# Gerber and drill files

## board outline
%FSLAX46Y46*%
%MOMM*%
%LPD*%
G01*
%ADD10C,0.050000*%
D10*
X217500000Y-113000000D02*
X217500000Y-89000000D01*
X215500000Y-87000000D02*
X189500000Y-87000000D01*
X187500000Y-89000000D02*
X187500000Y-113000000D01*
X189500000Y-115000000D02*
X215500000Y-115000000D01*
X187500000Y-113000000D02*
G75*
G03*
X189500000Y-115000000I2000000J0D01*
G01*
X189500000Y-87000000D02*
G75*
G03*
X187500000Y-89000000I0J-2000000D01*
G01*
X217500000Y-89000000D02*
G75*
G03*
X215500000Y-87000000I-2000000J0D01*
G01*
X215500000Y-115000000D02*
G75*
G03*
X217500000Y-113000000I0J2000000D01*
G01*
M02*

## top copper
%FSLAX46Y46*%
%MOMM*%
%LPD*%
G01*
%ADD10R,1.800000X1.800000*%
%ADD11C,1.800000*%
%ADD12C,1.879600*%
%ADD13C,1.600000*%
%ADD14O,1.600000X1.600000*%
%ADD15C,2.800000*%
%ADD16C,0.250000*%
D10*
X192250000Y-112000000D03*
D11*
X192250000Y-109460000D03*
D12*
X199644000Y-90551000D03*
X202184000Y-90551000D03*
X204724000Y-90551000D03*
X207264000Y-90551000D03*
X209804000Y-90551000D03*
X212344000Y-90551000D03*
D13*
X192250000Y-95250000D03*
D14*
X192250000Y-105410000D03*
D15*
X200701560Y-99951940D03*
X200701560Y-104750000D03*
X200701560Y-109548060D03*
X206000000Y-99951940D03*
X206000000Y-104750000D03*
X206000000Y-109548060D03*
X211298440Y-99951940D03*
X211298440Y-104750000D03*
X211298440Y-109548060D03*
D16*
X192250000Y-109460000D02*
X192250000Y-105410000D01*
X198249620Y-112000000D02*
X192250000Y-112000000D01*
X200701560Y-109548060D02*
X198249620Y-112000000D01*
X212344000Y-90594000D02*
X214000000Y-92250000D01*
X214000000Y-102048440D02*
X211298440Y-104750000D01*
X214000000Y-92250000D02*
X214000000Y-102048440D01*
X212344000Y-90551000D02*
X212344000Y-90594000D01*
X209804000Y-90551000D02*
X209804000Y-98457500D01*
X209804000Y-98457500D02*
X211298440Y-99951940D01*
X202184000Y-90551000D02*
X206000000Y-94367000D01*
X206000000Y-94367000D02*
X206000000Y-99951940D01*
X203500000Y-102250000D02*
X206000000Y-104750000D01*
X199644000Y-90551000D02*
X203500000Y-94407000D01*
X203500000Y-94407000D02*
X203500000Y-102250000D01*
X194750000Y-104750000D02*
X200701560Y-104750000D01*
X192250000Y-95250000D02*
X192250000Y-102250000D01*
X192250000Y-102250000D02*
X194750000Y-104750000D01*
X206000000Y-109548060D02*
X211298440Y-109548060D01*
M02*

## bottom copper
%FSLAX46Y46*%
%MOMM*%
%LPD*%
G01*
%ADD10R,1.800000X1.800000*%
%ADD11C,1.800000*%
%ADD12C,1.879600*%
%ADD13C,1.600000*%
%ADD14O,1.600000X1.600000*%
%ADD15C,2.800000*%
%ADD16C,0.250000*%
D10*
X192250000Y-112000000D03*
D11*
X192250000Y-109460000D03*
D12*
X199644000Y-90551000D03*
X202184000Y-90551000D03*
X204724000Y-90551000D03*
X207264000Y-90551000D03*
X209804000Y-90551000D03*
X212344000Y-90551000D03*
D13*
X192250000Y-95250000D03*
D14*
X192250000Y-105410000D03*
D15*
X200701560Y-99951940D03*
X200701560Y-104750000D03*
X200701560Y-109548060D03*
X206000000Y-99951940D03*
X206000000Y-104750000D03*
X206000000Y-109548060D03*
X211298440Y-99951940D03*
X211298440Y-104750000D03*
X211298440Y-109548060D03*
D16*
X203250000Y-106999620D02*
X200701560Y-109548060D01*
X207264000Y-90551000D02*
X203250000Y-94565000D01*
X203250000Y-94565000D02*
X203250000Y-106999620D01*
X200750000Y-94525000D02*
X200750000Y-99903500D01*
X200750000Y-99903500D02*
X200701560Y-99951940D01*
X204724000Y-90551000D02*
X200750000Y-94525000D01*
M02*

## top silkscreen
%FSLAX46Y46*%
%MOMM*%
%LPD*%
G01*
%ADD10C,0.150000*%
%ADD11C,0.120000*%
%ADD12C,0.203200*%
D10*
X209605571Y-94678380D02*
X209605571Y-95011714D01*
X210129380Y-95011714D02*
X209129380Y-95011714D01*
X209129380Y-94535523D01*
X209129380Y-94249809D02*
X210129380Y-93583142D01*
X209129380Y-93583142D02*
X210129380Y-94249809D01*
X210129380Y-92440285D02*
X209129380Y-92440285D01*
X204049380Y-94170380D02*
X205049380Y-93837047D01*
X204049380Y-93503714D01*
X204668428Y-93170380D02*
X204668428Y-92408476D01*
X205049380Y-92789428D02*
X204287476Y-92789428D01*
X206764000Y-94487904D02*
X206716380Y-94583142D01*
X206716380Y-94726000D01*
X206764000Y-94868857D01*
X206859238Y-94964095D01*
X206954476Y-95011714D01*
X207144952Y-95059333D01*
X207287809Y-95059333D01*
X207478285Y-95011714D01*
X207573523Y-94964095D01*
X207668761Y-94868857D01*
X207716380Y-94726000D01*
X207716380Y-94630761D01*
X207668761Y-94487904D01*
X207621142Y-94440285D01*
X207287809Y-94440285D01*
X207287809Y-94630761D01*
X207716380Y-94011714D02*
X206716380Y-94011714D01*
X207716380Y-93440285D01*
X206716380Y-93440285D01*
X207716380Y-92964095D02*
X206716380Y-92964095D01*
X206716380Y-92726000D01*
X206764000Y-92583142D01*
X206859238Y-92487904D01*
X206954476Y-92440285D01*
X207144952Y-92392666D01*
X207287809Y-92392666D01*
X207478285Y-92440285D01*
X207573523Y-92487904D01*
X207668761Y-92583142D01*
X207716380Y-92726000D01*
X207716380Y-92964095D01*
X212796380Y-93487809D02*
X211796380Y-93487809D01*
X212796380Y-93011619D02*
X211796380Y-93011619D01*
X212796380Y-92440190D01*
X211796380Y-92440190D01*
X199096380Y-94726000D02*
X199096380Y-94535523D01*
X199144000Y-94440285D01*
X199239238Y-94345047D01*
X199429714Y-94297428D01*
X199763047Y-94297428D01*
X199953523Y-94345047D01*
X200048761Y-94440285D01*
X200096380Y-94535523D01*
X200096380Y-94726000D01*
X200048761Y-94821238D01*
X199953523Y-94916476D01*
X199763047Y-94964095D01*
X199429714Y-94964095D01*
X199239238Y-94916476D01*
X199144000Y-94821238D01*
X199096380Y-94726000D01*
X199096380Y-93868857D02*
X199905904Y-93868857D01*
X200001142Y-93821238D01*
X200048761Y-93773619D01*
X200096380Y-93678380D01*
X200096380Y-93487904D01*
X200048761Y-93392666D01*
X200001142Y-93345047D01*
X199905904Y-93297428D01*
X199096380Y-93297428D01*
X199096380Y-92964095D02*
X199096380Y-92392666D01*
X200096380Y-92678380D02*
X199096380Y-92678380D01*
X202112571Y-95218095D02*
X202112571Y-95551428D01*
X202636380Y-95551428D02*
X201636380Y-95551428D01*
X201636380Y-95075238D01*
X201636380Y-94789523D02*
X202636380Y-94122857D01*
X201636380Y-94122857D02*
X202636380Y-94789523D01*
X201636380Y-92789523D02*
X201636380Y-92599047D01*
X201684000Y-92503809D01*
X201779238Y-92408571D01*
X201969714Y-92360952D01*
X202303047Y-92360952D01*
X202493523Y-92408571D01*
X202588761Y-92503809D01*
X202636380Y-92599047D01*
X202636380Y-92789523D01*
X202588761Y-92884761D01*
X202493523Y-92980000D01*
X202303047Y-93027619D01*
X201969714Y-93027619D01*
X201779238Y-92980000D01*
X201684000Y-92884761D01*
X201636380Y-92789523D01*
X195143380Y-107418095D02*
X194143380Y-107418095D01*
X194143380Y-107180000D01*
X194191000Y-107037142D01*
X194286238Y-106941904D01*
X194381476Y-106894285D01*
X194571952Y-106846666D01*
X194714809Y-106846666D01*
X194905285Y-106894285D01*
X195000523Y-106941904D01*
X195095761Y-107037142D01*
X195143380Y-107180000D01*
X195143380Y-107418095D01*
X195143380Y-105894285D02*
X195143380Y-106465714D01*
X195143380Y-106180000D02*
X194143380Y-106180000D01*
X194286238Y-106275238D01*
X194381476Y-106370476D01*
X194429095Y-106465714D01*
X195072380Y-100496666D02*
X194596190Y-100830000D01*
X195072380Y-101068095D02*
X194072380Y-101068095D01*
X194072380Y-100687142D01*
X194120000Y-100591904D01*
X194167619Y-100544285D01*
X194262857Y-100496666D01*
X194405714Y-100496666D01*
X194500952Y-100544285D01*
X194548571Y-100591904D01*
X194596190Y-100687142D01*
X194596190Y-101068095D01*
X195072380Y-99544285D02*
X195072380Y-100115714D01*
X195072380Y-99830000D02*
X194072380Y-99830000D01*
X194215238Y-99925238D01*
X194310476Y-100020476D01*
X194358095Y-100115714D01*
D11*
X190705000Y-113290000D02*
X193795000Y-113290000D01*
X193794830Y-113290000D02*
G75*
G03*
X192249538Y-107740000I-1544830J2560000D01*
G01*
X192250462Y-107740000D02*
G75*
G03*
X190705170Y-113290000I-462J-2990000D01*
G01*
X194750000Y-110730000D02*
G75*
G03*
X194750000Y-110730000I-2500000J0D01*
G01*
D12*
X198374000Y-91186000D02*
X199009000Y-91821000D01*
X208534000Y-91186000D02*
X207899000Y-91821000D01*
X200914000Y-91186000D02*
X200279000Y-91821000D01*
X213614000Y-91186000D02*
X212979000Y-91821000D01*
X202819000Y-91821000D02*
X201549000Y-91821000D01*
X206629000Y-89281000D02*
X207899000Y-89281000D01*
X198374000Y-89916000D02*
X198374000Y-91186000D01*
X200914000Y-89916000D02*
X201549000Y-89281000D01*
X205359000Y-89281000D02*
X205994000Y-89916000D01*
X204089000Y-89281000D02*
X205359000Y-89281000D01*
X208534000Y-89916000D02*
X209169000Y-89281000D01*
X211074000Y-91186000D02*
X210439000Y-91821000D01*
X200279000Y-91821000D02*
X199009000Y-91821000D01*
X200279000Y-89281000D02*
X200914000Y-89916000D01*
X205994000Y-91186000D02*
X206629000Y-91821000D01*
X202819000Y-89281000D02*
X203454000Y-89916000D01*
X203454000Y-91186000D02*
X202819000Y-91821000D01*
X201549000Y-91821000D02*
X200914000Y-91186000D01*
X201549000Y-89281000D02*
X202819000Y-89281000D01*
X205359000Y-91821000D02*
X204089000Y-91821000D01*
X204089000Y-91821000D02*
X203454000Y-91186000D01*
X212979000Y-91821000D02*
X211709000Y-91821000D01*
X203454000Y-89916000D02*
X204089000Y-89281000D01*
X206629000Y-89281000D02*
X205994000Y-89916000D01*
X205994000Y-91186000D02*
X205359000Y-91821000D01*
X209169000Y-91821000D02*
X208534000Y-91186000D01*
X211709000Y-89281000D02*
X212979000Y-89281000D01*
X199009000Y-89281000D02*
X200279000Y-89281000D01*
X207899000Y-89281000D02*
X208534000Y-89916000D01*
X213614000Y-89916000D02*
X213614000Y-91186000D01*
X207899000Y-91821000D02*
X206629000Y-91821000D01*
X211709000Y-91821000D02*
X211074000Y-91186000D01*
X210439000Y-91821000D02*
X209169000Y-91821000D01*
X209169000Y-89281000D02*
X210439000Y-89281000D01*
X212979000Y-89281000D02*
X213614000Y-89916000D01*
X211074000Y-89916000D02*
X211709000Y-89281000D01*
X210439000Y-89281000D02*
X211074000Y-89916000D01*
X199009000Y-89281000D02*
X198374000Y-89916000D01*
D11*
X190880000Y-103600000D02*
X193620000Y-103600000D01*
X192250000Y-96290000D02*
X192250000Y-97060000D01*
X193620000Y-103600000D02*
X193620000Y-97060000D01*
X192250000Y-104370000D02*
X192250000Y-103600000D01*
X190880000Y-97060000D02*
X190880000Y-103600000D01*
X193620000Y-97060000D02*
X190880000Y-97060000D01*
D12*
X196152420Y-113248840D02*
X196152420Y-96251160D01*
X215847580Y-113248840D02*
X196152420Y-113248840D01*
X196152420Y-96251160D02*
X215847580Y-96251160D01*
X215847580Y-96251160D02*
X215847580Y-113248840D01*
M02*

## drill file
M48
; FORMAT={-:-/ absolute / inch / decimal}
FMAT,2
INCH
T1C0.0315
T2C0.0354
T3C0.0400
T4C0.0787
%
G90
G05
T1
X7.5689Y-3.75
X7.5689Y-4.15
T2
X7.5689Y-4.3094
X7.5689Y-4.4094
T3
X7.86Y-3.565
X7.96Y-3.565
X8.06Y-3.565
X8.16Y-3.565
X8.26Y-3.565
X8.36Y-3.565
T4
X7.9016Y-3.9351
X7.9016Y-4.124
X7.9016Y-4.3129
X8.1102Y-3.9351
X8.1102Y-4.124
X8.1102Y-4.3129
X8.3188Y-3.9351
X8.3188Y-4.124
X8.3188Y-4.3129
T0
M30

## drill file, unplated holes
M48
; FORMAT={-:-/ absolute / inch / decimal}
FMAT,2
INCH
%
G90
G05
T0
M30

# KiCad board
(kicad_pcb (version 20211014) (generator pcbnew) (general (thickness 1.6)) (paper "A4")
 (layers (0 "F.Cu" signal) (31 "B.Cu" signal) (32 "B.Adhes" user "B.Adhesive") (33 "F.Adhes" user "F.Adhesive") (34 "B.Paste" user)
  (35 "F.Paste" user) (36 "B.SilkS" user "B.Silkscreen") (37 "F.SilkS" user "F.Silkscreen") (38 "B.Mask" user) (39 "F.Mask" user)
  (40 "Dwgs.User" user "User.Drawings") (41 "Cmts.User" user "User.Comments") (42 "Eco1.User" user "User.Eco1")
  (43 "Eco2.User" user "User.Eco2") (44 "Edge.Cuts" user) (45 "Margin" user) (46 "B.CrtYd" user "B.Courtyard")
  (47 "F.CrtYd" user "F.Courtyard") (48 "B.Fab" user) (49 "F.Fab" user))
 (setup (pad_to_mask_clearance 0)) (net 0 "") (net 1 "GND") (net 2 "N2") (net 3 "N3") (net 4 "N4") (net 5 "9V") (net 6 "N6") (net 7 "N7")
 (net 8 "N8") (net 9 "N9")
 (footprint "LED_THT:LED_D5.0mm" (layer "F.Cu") (at 192.25 112 90)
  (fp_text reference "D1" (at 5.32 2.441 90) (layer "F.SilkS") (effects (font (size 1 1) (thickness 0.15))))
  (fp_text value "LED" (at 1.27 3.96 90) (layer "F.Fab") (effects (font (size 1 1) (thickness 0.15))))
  (fp_line (start -1.29 -1.545) (end -1.29 1.545) (layer "F.SilkS") (width 0.12))
  (fp_arc (start 4.26 -0.000462) (mid 2.072002 2.880433) (end -1.29 1.54483) (layer "F.SilkS") (width 0.12))
  (fp_arc (start -1.29 -1.54483) (mid 2.072002 -2.880433) (end 4.26 0.000462) (layer "F.SilkS") (width 0.12))
  (fp_circle (center 1.27 0) (end 3.77 0) (layer "F.SilkS") (width 0.12) (fill none))
  (pad "1" thru_hole rect locked (at 0 0 90) (size 1.8 1.8) (drill 0.9) (layers *.Cu *.Mask) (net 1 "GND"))
  (pad "2" thru_hole circle locked (at 2.54 0 90) (size 1.8 1.8) (drill 0.9) (layers *.Cu *.Mask) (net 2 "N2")))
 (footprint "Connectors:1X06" (layer "F.Cu") (at 199.644 90.551)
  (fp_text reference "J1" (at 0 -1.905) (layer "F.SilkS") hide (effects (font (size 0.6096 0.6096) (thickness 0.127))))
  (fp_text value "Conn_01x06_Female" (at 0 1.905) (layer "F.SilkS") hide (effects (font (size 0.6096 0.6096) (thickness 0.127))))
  (fp_line (start -1.27 0.635) (end -0.635 1.27) (layer "F.SilkS") (width 0.2032))
  (fp_line (start 8.89 0.635) (end 8.255 1.27) (layer "F.SilkS") (width 0.2032))
  (fp_line (start 1.27 0.635) (end 0.635 1.27) (layer "F.SilkS") (width 0.2032))
  (fp_line (start 13.97 0.635) (end 13.335 1.27) (layer "F.SilkS") (width 0.2032))
  (fp_line (start 3.175 1.27) (end 1.905 1.27) (layer "F.SilkS") (width 0.2032))
  (fp_line (start 6.985 -1.27) (end 8.255 -1.27) (layer "F.SilkS") (width 0.2032))
  (fp_line (start -1.27 -0.635) (end -1.27 0.635) (layer "F.SilkS") (width 0.2032))
  (fp_line (start 1.27 -0.635) (end 1.905 -1.27) (layer "F.SilkS") (width 0.2032))
  (fp_line (start 5.715 -1.27) (end 6.35 -0.635) (layer "F.SilkS") (width 0.2032))
  (fp_line (start 4.445 -1.27) (end 5.715 -1.27) (layer "F.SilkS") (width 0.2032))
  (fp_line (start 8.89 -0.635) (end 9.525 -1.27) (layer "F.SilkS") (width 0.2032))
  (fp_line (start 11.43 0.635) (end 10.795 1.27) (layer "F.SilkS") (width 0.2032))
  (fp_line (start 0.635 1.27) (end -0.635 1.27) (layer "F.SilkS") (width 0.2032))
  (fp_line (start 0.635 -1.27) (end 1.27 -0.635) (layer "F.SilkS") (width 0.2032))
  (fp_line (start 6.35 0.635) (end 6.985 1.27) (layer "F.SilkS") (width 0.2032))
  (fp_line (start 3.175 -1.27) (end 3.81 -0.635) (layer "F.SilkS") (width 0.2032))
  (fp_line (start 3.81 0.635) (end 3.175 1.27) (layer "F.SilkS") (width 0.2032))
  (fp_line (start 1.905 1.27) (end 1.27 0.635) (layer "F.SilkS") (width 0.2032))
  (fp_line (start 1.905 -1.27) (end 3.175 -1.27) (layer "F.SilkS") (width 0.2032))
  (fp_line (start 5.715 1.27) (end 4.445 1.27) (layer "F.SilkS") (width 0.2032))
  (fp_line (start 4.445 1.27) (end 3.81 0.635) (layer "F.SilkS") (width 0.2032))
  (fp_line (start 13.335 1.27) (end 12.065 1.27) (layer "F.SilkS") (width 0.2032))
  (fp_line (start 3.81 -0.635) (end 4.445 -1.27) (layer "F.SilkS") (width 0.2032))
  (fp_line (start 6.985 -1.27) (end 6.35 -0.635) (layer "F.SilkS") (width 0.2032))
  (fp_line (start 6.35 0.635) (end 5.715 1.27) (layer "F.SilkS") (width 0.2032))
  (fp_line (start 9.525 1.27) (end 8.89 0.635) (layer "F.SilkS") (width 0.2032))
  (fp_line (start 12.065 -1.27) (end 13.335 -1.27) (layer "F.SilkS") (width 0.2032))
  (fp_line (start -0.635 -1.27) (end 0.635 -1.27) (layer "F.SilkS") (width 0.2032))
  (fp_line (start 8.255 -1.27) (end 8.89 -0.635) (layer "F.SilkS") (width 0.2032))
  (fp_line (start 13.97 -0.635) (end 13.97 0.635) (layer "F.SilkS") (width 0.2032))
  (fp_line (start 8.255 1.27) (end 6.985 1.27) (layer "F.SilkS") (width 0.2032))
  (fp_line (start 12.065 1.27) (end 11.43 0.635) (layer "F.SilkS") (width 0.2032))
  (fp_line (start 10.795 1.27) (end 9.525 1.27) (layer "F.SilkS") (width 0.2032))
  (fp_line (start 9.525 -1.27) (end 10.795 -1.27) (layer "F.SilkS") (width 0.2032))
  (fp_line (start 13.335 -1.27) (end 13.97 -0.635) (layer "F.SilkS") (width 0.2032))
  (fp_line (start 11.43 -0.635) (end 12.065 -1.27) (layer "F.SilkS") (width 0.2032))
  (fp_line (start 10.795 -1.27) (end 11.43 -0.635) (layer "F.SilkS") (width 0.2032))
  (fp_line (start -0.635 -1.27) (end -1.27 -0.635) (layer "F.SilkS") (width 0.2032))
  (pad "1" thru_hole circle locked (at 0 0) (size 1.8796 1.8796) (drill 1.016) (layers *.Cu *.Mask) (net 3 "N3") (solder_mask_margin 0.1016))
  (pad "2" thru_hole circle locked (at 2.54 0) (size 1.8796 1.8796) (drill 1.016) (layers *.Cu *.Mask) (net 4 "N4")
   (solder_mask_margin 0.1016))
  (pad "3" thru_hole circle locked (at 5.08 0) (size 1.8796 1.8796) (drill 1.016) (layers *.Cu *.Mask) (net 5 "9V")
   (solder_mask_margin 0.1016))
  (pad "4" thru_hole circle locked (at 7.62 0) (size 1.8796 1.8796) (drill 1.016) (layers *.Cu *.Mask) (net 1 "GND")
   (solder_mask_margin 0.1016))
  (pad "5" thru_hole circle locked (at 10.16 0) (size 1.8796 1.8796) (drill 1.016) (layers *.Cu *.Mask) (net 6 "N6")
   (solder_mask_margin 0.1016))
  (pad "6" thru_hole circle locked (at 12.7 0) (size 1.8796 1.8796) (drill 1.016) (layers *.Cu *.Mask) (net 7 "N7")
   (solder_mask_margin 0.1016)))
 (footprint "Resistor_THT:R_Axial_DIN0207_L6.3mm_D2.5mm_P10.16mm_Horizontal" (layer "F.Cu") (at 192.25 95.25 -90)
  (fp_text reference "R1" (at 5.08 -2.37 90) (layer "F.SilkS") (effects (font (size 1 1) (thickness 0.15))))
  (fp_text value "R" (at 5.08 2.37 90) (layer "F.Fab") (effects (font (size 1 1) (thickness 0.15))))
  (fp_line (start 8.35 1.37) (end 8.35 -1.37) (layer "F.SilkS") (width 0.12))
  (fp_line (start 1.04 0) (end 1.81 0) (layer "F.SilkS") (width 0.12))
  (fp_line (start 8.35 -1.37) (end 1.81 -1.37) (layer "F.SilkS") (width 0.12))
  (fp_line (start 9.12 0) (end 8.35 0) (layer "F.SilkS") (width 0.12))
  (fp_line (start 1.81 1.37) (end 8.35 1.37) (layer "F.SilkS") (width 0.12))
  (fp_line (start 1.81 -1.37) (end 1.81 1.37) (layer "F.SilkS") (width 0.12))
  (pad "1" thru_hole circle locked (at 0 0 270) (size 1.6 1.6) (drill 0.8) (layers *.Cu *.Mask) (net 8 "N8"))
  (pad "2" thru_hole oval locked (at 10.16 0 270) (size 1.6 1.6) (drill 0.8) (layers *.Cu *.Mask) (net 2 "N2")))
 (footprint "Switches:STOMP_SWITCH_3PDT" (layer "F.Cu") (at 206 104.75)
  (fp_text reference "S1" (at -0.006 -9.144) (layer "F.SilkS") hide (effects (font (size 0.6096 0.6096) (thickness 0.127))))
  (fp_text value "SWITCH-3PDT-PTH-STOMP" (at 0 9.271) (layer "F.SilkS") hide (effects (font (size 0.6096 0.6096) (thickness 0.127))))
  (fp_line (start -9.84758 8.49884) (end -9.84758 -8.49884) (layer "F.SilkS") (width 0.2032))
  (fp_line (start 9.84758 8.49884) (end -9.84758 8.49884) (layer "F.SilkS") (width 0.2032))
  (fp_line (start -9.84758 -8.49884) (end 9.84758 -8.49884) (layer "F.SilkS") (width 0.2032))
  (fp_line (start 9.84758 -8.49884) (end 9.84758 8.49884) (layer "F.SilkS") (width 0.2032))
  (pad "P$1" thru_hole circle (at -5.29844 -4.79806) (size 2.8 2.8) (drill 2) (layers *.Cu *.Mask) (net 5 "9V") (solder_mask_margin 0.1016))
  (pad "P$2" thru_hole circle (at -5.29844 0) (size 2.8 2.8) (drill 2) (layers *.Cu *.Mask) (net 8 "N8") (solder_mask_margin 0.1016))
  (pad "P$3" thru_hole circle (at -5.29844 4.79806) (size 2.8 2.8) (drill 2) (layers *.Cu *.Mask) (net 1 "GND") (solder_mask_margin 0.1016))
  (pad "P$4" thru_hole circle (at 0 -4.79806) (size 2.8 2.8) (drill 2) (layers *.Cu *.Mask) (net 4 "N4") (solder_mask_margin 0.1016))
  (pad "P$5" thru_hole circle (at 0 0) (size 2.8 2.8) (drill 2) (layers *.Cu *.Mask) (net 3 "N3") (solder_mask_margin 0.1016))
  (pad "P$6" thru_hole circle (at 0 4.79806) (size 2.8 2.8) (drill 2) (layers *.Cu *.Mask) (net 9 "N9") (solder_mask_margin 0.1016))
  (pad "P$7" thru_hole circle (at 5.29844 -4.79806) (size 2.8 2.8) (drill 2) (layers *.Cu *.Mask) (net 6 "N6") (solder_mask_margin 0.1016))
  (pad "P$8" thru_hole circle (at 5.29844 0) (size 2.8 2.8) (drill 2) (layers *.Cu *.Mask) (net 7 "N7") (solder_mask_margin 0.1016))
  (pad "P$9" thru_hole circle (at 5.29844 4.79806) (size 2.8 2.8) (drill 2) (layers *.Cu *.Mask) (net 9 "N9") (solder_mask_margin 0.1016)))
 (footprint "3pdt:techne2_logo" (layer "B.Cu") (at 212.25 95.1 180)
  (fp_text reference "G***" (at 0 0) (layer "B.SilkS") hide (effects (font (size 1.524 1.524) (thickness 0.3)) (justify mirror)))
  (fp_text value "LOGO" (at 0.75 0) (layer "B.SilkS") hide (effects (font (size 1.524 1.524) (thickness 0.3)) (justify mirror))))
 (gr_line (start 217.5 113) (end 217.5 89) (layer "Edge.Cuts") (width 0.05))
 (gr_line (start 215.5 87) (end 189.5 87) (layer "Edge.Cuts") (width 0.05))
 (gr_line (start 187.5 89) (end 187.5 113) (layer "Edge.Cuts") (width 0.05))
 (gr_line (start 189.5 115) (end 215.5 115) (layer "Edge.Cuts") (width 0.05))
 (gr_arc (start 189.5 115) (mid 188.085786 114.414214) (end 187.5 113) (layer "Edge.Cuts") (width 0.05))
 (gr_arc (start 187.5 89) (mid 188.085786 87.585786) (end 189.5 87) (layer "Edge.Cuts") (width 0.05))
 (gr_arc (start 215.5 87) (mid 216.914214 87.585786) (end 217.5 89) (layer "Edge.Cuts") (width 0.05))
 (gr_arc (start 217.5 113) (mid 216.914214 114.414214) (end 215.5 115) (layer "Edge.Cuts") (width 0.05))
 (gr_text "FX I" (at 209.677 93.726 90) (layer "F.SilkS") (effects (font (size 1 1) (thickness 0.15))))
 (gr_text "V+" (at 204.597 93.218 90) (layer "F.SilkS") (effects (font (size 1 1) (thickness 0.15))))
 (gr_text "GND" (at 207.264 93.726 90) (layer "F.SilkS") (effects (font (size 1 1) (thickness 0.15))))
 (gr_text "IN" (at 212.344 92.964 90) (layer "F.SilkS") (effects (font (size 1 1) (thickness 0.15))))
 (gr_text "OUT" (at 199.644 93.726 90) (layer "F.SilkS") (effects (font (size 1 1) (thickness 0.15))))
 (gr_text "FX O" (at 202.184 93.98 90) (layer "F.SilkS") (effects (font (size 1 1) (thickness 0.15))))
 (segment (start 192.25 109.46) (end 192.25 105.41) (width 0.25) (layer "F.Cu") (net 2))
 (segment (start 198.24962 112) (end 192.25 112) (width 0.25) (layer "F.Cu") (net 1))
 (segment (start 200.70156 109.54806) (end 198.24962 112) (width 0.25) (layer "F.Cu") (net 1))
 (segment (start 203.25 106.99962) (end 200.70156 109.54806) (width 0.25) (layer "B.Cu") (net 1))
 (segment (start 207.264 90.551) (end 203.25 94.565) (width 0.25) (layer "B.Cu") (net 1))
 (segment (start 203.25 94.565) (end 203.25 106.99962) (width 0.25) (layer "B.Cu") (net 1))
 (segment (start 212.344 90.594) (end 214 92.25) (width 0.25) (layer "F.Cu") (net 7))
 (segment (start 214 102.04844) (end 211.29844 104.75) (width 0.25) (layer "F.Cu") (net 7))
 (segment (start 214 92.25) (end 214 102.04844) (width 0.25) (layer "F.Cu") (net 7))
 (segment (start 212.344 90.551) (end 212.344 90.594) (width 0.25) (layer "F.Cu") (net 7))
 (segment (start 209.804 90.551) (end 209.804 98.4575) (width 0.25) (layer "F.Cu") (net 6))
 (segment (start 209.804 98.4575) (end 211.29844 99.95194) (width 0.25) (layer "F.Cu") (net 6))
 (segment (start 200.75 94.525) (end 200.75 99.9035) (width 0.25) (layer "B.Cu") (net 5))
 (segment (start 200.75 99.9035) (end 200.70156 99.95194) (width 0.25) (layer "B.Cu") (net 5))
 (segment (start 204.724 90.551) (end 200.75 94.525) (width 0.25) (layer "B.Cu") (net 5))
 (segment (start 202.184 90.551) (end 206 94.367) (width 0.25) (layer "F.Cu") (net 4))
 (segment (start 206 94.367) (end 206 99.95194) (width 0.25) (layer "F.Cu") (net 4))
 (segment (start 203.5 102.25) (end 206 104.75) (width 0.25) (layer "F.Cu") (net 3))
 (segment (start 199.644 90.551) (end 203.5 94.407) (width 0.25) (layer "F.Cu") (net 3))
 (segment (start 203.5 94.407) (end 203.5 102.25) (width 0.25) (layer "F.Cu") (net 3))
 (segment (start 194.75 104.75) (end 200.70156 104.75) (width 0.25) (layer "F.Cu") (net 8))
 (segment (start 192.25 95.25) (end 192.25 102.25) (width 0.25) (layer "F.Cu") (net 8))
 (segment (start 192.25 102.25) (end 194.75 104.75) (width 0.25) (layer "F.Cu") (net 8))
 (segment (start 206 109.54806) (end 211.29844 109.54806) (width 0.25) (layer "F.Cu") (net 9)))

